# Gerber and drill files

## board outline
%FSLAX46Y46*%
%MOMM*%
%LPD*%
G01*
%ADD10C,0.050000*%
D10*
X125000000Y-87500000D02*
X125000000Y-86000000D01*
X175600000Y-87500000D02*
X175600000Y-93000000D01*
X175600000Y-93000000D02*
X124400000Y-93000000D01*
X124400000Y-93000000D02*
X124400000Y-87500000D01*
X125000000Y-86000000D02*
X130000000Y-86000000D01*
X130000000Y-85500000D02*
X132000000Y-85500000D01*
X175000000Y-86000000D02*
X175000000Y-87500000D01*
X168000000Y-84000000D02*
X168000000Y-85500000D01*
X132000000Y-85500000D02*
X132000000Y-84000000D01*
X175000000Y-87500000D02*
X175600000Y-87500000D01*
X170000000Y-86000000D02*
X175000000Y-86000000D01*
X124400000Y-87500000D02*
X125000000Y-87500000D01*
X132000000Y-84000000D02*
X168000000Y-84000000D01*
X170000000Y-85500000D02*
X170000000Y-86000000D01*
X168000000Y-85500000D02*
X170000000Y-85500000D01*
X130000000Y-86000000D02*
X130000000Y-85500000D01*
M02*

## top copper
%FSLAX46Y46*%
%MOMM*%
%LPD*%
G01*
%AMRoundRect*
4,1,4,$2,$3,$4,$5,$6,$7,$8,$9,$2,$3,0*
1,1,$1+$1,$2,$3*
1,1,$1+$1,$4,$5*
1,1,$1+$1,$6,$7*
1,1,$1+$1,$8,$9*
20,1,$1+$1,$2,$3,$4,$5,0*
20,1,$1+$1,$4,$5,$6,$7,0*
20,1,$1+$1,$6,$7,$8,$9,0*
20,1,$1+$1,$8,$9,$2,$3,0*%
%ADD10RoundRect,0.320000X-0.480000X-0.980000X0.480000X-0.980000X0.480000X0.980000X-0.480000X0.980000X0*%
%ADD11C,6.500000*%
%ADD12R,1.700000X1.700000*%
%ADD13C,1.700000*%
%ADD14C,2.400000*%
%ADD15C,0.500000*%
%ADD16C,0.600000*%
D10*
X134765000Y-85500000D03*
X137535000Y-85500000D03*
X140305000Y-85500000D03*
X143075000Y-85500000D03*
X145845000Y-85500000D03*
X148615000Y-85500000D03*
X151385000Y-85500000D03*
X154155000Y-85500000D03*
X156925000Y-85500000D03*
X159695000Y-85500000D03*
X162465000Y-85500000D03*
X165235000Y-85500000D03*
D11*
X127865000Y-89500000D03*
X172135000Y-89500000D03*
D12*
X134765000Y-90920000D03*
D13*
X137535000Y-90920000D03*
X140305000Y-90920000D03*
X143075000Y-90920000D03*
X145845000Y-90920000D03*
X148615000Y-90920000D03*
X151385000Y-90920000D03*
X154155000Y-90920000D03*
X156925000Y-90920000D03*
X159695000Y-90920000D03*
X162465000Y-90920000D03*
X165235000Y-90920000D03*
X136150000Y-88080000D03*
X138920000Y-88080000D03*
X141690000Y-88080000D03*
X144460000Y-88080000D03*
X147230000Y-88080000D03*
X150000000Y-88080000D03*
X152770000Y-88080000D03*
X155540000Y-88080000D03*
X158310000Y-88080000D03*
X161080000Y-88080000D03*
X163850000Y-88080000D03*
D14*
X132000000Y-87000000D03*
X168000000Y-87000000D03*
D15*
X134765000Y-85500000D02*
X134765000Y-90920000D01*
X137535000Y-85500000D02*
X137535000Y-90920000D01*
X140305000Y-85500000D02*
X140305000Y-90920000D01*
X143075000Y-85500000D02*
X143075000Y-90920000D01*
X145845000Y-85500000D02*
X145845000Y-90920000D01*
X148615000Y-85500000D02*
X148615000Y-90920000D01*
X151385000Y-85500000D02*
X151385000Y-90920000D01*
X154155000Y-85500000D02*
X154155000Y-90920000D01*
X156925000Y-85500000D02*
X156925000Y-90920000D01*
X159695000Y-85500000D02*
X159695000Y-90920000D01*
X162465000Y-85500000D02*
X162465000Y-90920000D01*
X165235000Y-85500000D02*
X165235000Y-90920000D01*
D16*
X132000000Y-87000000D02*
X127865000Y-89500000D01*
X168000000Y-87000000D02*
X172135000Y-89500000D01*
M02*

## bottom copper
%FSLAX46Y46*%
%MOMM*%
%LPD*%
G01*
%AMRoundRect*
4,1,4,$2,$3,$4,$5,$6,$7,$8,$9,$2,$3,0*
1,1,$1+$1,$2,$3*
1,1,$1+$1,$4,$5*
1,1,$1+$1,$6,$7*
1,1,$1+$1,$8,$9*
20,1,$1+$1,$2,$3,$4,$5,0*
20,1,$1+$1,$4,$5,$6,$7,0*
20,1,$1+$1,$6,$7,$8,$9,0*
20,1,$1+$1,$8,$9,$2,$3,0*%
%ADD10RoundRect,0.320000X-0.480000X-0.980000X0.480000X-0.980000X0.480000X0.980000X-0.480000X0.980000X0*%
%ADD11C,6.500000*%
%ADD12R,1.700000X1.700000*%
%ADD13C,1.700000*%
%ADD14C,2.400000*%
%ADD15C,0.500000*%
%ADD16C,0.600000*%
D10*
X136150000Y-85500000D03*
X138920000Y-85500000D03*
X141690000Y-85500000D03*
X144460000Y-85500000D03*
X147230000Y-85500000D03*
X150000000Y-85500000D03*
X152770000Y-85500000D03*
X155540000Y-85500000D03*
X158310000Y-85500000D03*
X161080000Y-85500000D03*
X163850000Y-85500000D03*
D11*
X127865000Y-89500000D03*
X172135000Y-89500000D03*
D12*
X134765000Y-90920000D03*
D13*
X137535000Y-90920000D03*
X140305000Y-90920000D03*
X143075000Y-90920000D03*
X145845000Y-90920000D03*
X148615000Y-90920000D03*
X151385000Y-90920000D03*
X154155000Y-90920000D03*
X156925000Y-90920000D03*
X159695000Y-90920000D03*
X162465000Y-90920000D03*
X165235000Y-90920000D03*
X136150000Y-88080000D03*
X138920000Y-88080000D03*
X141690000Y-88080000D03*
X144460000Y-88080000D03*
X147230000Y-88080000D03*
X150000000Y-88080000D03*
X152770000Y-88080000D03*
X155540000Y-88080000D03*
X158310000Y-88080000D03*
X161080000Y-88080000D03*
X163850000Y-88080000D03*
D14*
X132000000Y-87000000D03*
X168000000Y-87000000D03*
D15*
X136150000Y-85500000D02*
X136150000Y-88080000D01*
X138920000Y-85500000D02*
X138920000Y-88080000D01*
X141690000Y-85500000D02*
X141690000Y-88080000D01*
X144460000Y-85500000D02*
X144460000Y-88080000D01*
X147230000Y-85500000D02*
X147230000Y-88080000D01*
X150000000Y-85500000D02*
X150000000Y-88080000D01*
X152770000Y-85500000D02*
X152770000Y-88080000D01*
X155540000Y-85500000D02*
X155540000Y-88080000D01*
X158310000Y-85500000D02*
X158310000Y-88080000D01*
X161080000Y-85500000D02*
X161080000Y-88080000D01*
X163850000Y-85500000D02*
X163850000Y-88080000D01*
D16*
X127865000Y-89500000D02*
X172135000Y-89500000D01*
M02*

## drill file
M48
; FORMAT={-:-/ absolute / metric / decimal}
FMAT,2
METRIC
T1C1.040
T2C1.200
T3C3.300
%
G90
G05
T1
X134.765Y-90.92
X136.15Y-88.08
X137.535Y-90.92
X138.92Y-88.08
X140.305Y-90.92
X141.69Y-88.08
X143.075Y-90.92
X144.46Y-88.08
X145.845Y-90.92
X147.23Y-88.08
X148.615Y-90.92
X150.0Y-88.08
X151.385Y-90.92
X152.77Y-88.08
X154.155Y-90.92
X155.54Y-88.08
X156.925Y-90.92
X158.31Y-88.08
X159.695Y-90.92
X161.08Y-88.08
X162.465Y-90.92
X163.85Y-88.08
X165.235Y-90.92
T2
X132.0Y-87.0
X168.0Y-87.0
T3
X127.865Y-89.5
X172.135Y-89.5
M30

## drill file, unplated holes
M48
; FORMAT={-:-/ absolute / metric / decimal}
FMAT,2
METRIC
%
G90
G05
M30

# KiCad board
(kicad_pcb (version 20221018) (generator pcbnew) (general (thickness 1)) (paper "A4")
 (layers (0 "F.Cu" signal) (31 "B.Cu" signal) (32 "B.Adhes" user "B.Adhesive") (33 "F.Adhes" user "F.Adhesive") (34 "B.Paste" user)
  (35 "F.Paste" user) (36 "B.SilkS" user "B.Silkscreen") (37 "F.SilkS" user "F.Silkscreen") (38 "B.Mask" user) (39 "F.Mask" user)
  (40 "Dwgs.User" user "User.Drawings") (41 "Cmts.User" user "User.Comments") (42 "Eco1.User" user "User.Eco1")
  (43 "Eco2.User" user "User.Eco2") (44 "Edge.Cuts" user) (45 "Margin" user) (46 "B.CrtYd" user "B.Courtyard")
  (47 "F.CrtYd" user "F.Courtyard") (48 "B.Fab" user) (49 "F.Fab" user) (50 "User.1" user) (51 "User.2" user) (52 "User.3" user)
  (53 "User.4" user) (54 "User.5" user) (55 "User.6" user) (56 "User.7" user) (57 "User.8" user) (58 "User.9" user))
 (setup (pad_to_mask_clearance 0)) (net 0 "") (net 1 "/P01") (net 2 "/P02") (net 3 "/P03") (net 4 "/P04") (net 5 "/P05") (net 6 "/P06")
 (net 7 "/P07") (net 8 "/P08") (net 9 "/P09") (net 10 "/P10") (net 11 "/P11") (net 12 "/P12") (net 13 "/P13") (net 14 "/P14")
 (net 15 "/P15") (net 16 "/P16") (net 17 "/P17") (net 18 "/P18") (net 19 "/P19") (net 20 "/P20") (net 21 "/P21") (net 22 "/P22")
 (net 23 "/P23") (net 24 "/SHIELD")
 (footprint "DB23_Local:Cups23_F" (layer "F.Cu") (at 150 80)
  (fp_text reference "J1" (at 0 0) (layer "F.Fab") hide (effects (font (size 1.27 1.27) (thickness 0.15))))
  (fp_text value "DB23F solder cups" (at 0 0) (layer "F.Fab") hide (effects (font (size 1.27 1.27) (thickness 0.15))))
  (pad "1" smd roundrect (at -15.235 5.5) (size 1.6 2.6) (layers "F.Cu" "F.Mask") (roundrect_rratio 0.2) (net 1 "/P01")
   (thermal_bridge_angle 45))
  (pad "2" smd roundrect (at -12.465 5.5) (size 1.6 2.6) (layers "F.Cu" "F.Mask") (roundrect_rratio 0.2) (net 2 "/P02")
   (thermal_bridge_angle 45))
  (pad "3" smd roundrect (at -9.695 5.5) (size 1.6 2.6) (layers "F.Cu" "F.Mask") (roundrect_rratio 0.2) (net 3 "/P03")
   (thermal_bridge_angle 45))
  (pad "4" smd roundrect (at -6.925 5.5) (size 1.6 2.6) (layers "F.Cu" "F.Mask") (roundrect_rratio 0.2) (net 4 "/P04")
   (thermal_bridge_angle 45))
  (pad "5" smd roundrect (at -4.155 5.5) (size 1.6 2.6) (layers "F.Cu" "F.Mask") (roundrect_rratio 0.2) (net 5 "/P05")
   (thermal_bridge_angle 45))
  (pad "6" smd roundrect (at -1.385 5.5) (size 1.6 2.6) (layers "F.Cu" "F.Mask") (roundrect_rratio 0.2) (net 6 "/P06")
   (thermal_bridge_angle 45))
  (pad "7" smd roundrect (at 1.385 5.5) (size 1.6 2.6) (layers "F.Cu" "F.Mask") (roundrect_rratio 0.2) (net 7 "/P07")
   (thermal_bridge_angle 45))
  (pad "8" smd roundrect (at 4.155 5.5) (size 1.6 2.6) (layers "F.Cu" "F.Mask") (roundrect_rratio 0.2) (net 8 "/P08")
   (thermal_bridge_angle 45))
  (pad "9" smd roundrect (at 6.925 5.5) (size 1.6 2.6) (layers "F.Cu" "F.Mask") (roundrect_rratio 0.2) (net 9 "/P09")
   (thermal_bridge_angle 45))
  (pad "10" smd roundrect (at 9.695 5.5) (size 1.6 2.6) (layers "F.Cu" "F.Mask") (roundrect_rratio 0.2) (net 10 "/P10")
   (thermal_bridge_angle 45))
  (pad "11" smd roundrect (at 12.465 5.5) (size 1.6 2.6) (layers "F.Cu" "F.Mask") (roundrect_rratio 0.2) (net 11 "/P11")
   (thermal_bridge_angle 45))
  (pad "12" smd roundrect (at 15.235 5.5) (size 1.6 2.6) (layers "F.Cu" "F.Mask") (roundrect_rratio 0.2) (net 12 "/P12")
   (thermal_bridge_angle 45))
  (pad "13" smd roundrect (at -13.85 5.5) (size 1.6 2.6) (layers "B.Cu" "B.Mask") (roundrect_rratio 0.2) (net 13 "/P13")
   (thermal_bridge_angle 45))
  (pad "14" smd roundrect (at -11.08 5.5) (size 1.6 2.6) (layers "B.Cu" "B.Mask") (roundrect_rratio 0.2) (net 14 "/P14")
   (thermal_bridge_angle 45))
  (pad "15" smd roundrect (at -8.31 5.5) (size 1.6 2.6) (layers "B.Cu" "B.Mask") (roundrect_rratio 0.2) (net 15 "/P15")
   (thermal_bridge_angle 45))
  (pad "16" smd roundrect (at -5.54 5.5) (size 1.6 2.6) (layers "B.Cu" "B.Mask") (roundrect_rratio 0.2) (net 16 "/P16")
   (thermal_bridge_angle 45))
  (pad "17" smd roundrect (at -2.77 5.5) (size 1.6 2.6) (layers "B.Cu" "B.Mask") (roundrect_rratio 0.2) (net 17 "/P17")
   (thermal_bridge_angle 45))
  (pad "18" smd roundrect (at 0 5.5) (size 1.6 2.6) (layers "B.Cu" "B.Mask") (roundrect_rratio 0.2) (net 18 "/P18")
   (thermal_bridge_angle 45))
  (pad "19" smd roundrect (at 2.77 5.5) (size 1.6 2.6) (layers "B.Cu" "B.Mask") (roundrect_rratio 0.2) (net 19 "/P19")
   (thermal_bridge_angle 45))
  (pad "20" smd roundrect (at 5.54 5.5) (size 1.6 2.6) (layers "B.Cu" "B.Mask") (roundrect_rratio 0.2) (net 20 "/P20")
   (thermal_bridge_angle 45))
  (pad "21" smd roundrect (at 8.31 5.5) (size 1.6 2.6) (layers "B.Cu" "B.Mask") (roundrect_rratio 0.2) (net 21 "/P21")
   (thermal_bridge_angle 45))
  (pad "22" smd roundrect (at 11.08 5.5) (size 1.6 2.6) (layers "B.Cu" "B.Mask") (roundrect_rratio 0.2) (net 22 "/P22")
   (thermal_bridge_angle 45))
  (pad "23" smd roundrect (at 13.85 5.5) (size 1.6 2.6) (layers "B.Cu" "B.Mask") (roundrect_rratio 0.2) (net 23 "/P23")
   (thermal_bridge_angle 45)))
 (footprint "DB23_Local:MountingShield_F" (layer "F.Cu") (at 150 80)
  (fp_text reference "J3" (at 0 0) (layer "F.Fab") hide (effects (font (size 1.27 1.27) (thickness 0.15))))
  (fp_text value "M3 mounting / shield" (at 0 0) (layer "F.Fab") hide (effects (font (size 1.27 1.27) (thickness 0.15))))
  (pad "1" thru_hole circle (at -22.135 9.5) (size 6.5 6.5) (drill 3.3) (layers "*.Cu" "*.Mask") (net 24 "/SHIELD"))
  (pad "2" thru_hole circle (at 22.135 9.5) (size 6.5 6.5) (drill 3.3) (layers "*.Cu" "*.Mask") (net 24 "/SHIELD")))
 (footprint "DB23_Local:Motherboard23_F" (layer "F.Cu") (at 150 80)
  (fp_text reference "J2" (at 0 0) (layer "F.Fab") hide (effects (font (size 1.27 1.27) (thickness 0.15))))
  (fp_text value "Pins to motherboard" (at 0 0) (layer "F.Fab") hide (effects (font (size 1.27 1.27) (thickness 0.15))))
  (pad "1" thru_hole rect (at -15.235 10.92) (size 1.7 1.7) (drill 1.04) (layers "*.Cu" "*.Mask") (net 1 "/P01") (thermal_bridge_angle 45))
  (pad "2" thru_hole circle (at -12.465 10.92) (size 1.7 1.7) (drill 1.04) (layers "*.Cu" "*.Mask") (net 2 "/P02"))
  (pad "3" thru_hole circle (at -9.695 10.92) (size 1.7 1.7) (drill 1.04) (layers "*.Cu" "*.Mask") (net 3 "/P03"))
  (pad "4" thru_hole circle (at -6.925 10.92) (size 1.7 1.7) (drill 1.04) (layers "*.Cu" "*.Mask") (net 4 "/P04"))
  (pad "5" thru_hole circle (at -4.155 10.92) (size 1.7 1.7) (drill 1.04) (layers "*.Cu" "*.Mask") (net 5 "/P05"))
  (pad "6" thru_hole circle (at -1.385 10.92) (size 1.7 1.7) (drill 1.04) (layers "*.Cu" "*.Mask") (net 6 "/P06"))
  (pad "7" thru_hole circle (at 1.385 10.92) (size 1.7 1.7) (drill 1.04) (layers "*.Cu" "*.Mask") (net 7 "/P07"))
  (pad "8" thru_hole circle (at 4.155 10.92) (size 1.7 1.7) (drill 1.04) (layers "*.Cu" "*.Mask") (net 8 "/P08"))
  (pad "9" thru_hole circle (at 6.925 10.92) (size 1.7 1.7) (drill 1.04) (layers "*.Cu" "*.Mask") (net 9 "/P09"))
  (pad "10" thru_hole circle (at 9.695 10.92) (size 1.7 1.7) (drill 1.04) (layers "*.Cu" "*.Mask") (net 10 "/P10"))
  (pad "11" thru_hole circle (at 12.465 10.92) (size 1.7 1.7) (drill 1.04) (layers "*.Cu" "*.Mask") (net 11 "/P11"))
  (pad "12" thru_hole circle (at 15.235 10.92) (size 1.7 1.7) (drill 1.04) (layers "*.Cu" "*.Mask") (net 12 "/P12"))
  (pad "13" thru_hole circle (at -13.85 8.08) (size 1.7 1.7) (drill 1.04) (layers "*.Cu" "*.Mask") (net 13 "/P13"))
  (pad "14" thru_hole circle (at -11.08 8.08) (size 1.7 1.7) (drill 1.04) (layers "*.Cu" "*.Mask") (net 14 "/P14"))
  (pad "15" thru_hole circle (at -8.31 8.08) (size 1.7 1.7) (drill 1.04) (layers "*.Cu" "*.Mask") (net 15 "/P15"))
  (pad "16" thru_hole circle (at -5.54 8.08) (size 1.7 1.7) (drill 1.04) (layers "*.Cu" "*.Mask") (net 16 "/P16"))
  (pad "17" thru_hole circle (at -2.77 8.08) (size 1.7 1.7) (drill 1.04) (layers "*.Cu" "*.Mask") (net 17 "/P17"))
  (pad "18" thru_hole circle (at 0 8.08) (size 1.7 1.7) (drill 1.04) (layers "*.Cu" "*.Mask") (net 18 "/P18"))
  (pad "19" thru_hole circle (at 2.77 8.08) (size 1.7 1.7) (drill 1.04) (layers "*.Cu" "*.Mask") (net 19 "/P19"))
  (pad "20" thru_hole circle (at 5.54 8.08) (size 1.7 1.7) (drill 1.04) (layers "*.Cu" "*.Mask") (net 20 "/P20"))
  (pad "21" thru_hole circle (at 8.31 8.08) (size 1.7 1.7) (drill 1.04) (layers "*.Cu" "*.Mask") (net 21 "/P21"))
  (pad "22" thru_hole circle (at 11.08 8.08) (size 1.7 1.7) (drill 1.04) (layers "*.Cu" "*.Mask") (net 22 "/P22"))
  (pad "23" thru_hole circle (at 13.85 8.08) (size 1.7 1.7) (drill 1.04) (layers "*.Cu" "*.Mask") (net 23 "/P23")))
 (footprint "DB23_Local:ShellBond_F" (layer "F.Cu") (at 150 80)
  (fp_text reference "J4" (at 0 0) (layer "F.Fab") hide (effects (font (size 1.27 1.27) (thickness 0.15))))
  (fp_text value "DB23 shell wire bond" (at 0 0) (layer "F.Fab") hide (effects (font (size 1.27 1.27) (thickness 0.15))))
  (pad "1" thru_hole circle (at -18 7) (size 2.4 2.4) (drill 1.2) (layers "*.Cu" "*.Mask") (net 24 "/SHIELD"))
  (pad "2" thru_hole circle (at 18 7) (size 2.4 2.4) (drill 1.2) (layers "*.Cu" "*.Mask") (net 24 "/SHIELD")))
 (gr_line (start 125 87.5) (end 125 86) (stroke (width 0.05) (type default)) (layer "Edge.Cuts"))
 (gr_line (start 175.6 87.5) (end 175.6 93) (stroke (width 0.05) (type default)) (layer "Edge.Cuts"))
 (gr_line (start 175.6 93) (end 124.4 93) (stroke (width 0.05) (type default)) (layer "Edge.Cuts"))
 (gr_line (start 124.4 93) (end 124.4 87.5) (stroke (width 0.05) (type default)) (layer "Edge.Cuts"))
 (gr_line (start 125 86) (end 130 86) (stroke (width 0.05) (type default)) (layer "Edge.Cuts"))
 (gr_line (start 130 85.5) (end 132 85.5) (stroke (width 0.05) (type default)) (layer "Edge.Cuts"))
 (gr_line (start 175 86) (end 175 87.5) (stroke (width 0.05) (type default)) (layer "Edge.Cuts"))
 (gr_line (start 168 84) (end 168 85.5) (stroke (width 0.05) (type default)) (layer "Edge.Cuts"))
 (gr_line (start 132 85.5) (end 132 84) (stroke (width 0.05) (type default)) (layer "Edge.Cuts"))
 (gr_line (start 175 87.5) (end 175.6 87.5) (stroke (width 0.05) (type default)) (layer "Edge.Cuts"))
 (gr_line (start 170 86) (end 175 86) (stroke (width 0.05) (type default)) (layer "Edge.Cuts"))
 (gr_line (start 124.4 87.5) (end 125 87.5) (stroke (width 0.05) (type default)) (layer "Edge.Cuts"))
 (gr_line (start 132 84) (end 168 84) (stroke (width 0.05) (type default)) (layer "Edge.Cuts"))
 (gr_line (start 170 85.5) (end 170 86) (stroke (width 0.05) (type default)) (layer "Edge.Cuts"))
 (gr_line (start 168 85.5) (end 170 85.5) (stroke (width 0.05) (type default)) (layer "Edge.Cuts"))
 (gr_line (start 130 86) (end 130 85.5) (stroke (width 0.05) (type default)) (layer "Edge.Cuts"))
 (segment (start 134.765 85.5) (end 134.765 90.92) (width 0.5) (layer "F.Cu") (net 1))
 (segment (start 137.535 85.5) (end 137.535 90.92) (width 0.5) (layer "F.Cu") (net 2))
 (segment (start 140.305 85.5) (end 140.305 90.92) (width 0.5) (layer "F.Cu") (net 3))
 (segment (start 143.075 85.5) (end 143.075 90.92) (width 0.5) (layer "F.Cu") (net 4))
 (segment (start 145.845 85.5) (end 145.845 90.92) (width 0.5) (layer "F.Cu") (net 5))
 (segment (start 148.615 85.5) (end 148.615 90.92) (width 0.5) (layer "F.Cu") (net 6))
 (segment (start 151.385 85.5) (end 151.385 90.92) (width 0.5) (layer "F.Cu") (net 7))
 (segment (start 154.155 85.5) (end 154.155 90.92) (width 0.5) (layer "F.Cu") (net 8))
 (segment (start 156.925 85.5) (end 156.925 90.92) (width 0.5) (layer "F.Cu") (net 9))
 (segment (start 159.695 85.5) (end 159.695 90.92) (width 0.5) (layer "F.Cu") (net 10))
 (segment (start 162.465 85.5) (end 162.465 90.92) (width 0.5) (layer "F.Cu") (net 11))
 (segment (start 165.235 85.5) (end 165.235 90.92) (width 0.5) (layer "F.Cu") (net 12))
 (segment (start 136.15 85.5) (end 136.15 88.08) (width 0.5) (layer "B.Cu") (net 13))
 (segment (start 138.92 85.5) (end 138.92 88.08) (width 0.5) (layer "B.Cu") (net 14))
 (segment (start 141.69 85.5) (end 141.69 88.08) (width 0.5) (layer "B.Cu") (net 15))
 (segment (start 144.46 85.5) (end 144.46 88.08) (width 0.5) (layer "B.Cu") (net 16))
 (segment (start 147.23 85.5) (end 147.23 88.08) (width 0.5) (layer "B.Cu") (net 17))
 (segment (start 150 85.5) (end 150 88.08) (width 0.5) (layer "B.Cu") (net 18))
 (segment (start 152.77 85.5) (end 152.77 88.08) (width 0.5) (layer "B.Cu") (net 19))
 (segment (start 155.54 85.5) (end 155.54 88.08) (width 0.5) (layer "B.Cu") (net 20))
 (segment (start 158.31 85.5) (end 158.31 88.08) (width 0.5) (layer "B.Cu") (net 21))
 (segment (start 161.08 85.5) (end 161.08 88.08) (width 0.5) (layer "B.Cu") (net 22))
 (segment (start 163.85 85.5) (end 163.85 88.08) (width 0.5) (layer "B.Cu") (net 23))
 (segment (start 132 87) (end 127.865 89.5) (width 0.6) (layer "F.Cu") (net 24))
 (segment (start 168 87) (end 172.135 89.5) (width 0.6) (layer "F.Cu") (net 24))
 (segment (start 127.865 89.5) (end 172.135 89.5) (width 0.6) (layer "B.Cu") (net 24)))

